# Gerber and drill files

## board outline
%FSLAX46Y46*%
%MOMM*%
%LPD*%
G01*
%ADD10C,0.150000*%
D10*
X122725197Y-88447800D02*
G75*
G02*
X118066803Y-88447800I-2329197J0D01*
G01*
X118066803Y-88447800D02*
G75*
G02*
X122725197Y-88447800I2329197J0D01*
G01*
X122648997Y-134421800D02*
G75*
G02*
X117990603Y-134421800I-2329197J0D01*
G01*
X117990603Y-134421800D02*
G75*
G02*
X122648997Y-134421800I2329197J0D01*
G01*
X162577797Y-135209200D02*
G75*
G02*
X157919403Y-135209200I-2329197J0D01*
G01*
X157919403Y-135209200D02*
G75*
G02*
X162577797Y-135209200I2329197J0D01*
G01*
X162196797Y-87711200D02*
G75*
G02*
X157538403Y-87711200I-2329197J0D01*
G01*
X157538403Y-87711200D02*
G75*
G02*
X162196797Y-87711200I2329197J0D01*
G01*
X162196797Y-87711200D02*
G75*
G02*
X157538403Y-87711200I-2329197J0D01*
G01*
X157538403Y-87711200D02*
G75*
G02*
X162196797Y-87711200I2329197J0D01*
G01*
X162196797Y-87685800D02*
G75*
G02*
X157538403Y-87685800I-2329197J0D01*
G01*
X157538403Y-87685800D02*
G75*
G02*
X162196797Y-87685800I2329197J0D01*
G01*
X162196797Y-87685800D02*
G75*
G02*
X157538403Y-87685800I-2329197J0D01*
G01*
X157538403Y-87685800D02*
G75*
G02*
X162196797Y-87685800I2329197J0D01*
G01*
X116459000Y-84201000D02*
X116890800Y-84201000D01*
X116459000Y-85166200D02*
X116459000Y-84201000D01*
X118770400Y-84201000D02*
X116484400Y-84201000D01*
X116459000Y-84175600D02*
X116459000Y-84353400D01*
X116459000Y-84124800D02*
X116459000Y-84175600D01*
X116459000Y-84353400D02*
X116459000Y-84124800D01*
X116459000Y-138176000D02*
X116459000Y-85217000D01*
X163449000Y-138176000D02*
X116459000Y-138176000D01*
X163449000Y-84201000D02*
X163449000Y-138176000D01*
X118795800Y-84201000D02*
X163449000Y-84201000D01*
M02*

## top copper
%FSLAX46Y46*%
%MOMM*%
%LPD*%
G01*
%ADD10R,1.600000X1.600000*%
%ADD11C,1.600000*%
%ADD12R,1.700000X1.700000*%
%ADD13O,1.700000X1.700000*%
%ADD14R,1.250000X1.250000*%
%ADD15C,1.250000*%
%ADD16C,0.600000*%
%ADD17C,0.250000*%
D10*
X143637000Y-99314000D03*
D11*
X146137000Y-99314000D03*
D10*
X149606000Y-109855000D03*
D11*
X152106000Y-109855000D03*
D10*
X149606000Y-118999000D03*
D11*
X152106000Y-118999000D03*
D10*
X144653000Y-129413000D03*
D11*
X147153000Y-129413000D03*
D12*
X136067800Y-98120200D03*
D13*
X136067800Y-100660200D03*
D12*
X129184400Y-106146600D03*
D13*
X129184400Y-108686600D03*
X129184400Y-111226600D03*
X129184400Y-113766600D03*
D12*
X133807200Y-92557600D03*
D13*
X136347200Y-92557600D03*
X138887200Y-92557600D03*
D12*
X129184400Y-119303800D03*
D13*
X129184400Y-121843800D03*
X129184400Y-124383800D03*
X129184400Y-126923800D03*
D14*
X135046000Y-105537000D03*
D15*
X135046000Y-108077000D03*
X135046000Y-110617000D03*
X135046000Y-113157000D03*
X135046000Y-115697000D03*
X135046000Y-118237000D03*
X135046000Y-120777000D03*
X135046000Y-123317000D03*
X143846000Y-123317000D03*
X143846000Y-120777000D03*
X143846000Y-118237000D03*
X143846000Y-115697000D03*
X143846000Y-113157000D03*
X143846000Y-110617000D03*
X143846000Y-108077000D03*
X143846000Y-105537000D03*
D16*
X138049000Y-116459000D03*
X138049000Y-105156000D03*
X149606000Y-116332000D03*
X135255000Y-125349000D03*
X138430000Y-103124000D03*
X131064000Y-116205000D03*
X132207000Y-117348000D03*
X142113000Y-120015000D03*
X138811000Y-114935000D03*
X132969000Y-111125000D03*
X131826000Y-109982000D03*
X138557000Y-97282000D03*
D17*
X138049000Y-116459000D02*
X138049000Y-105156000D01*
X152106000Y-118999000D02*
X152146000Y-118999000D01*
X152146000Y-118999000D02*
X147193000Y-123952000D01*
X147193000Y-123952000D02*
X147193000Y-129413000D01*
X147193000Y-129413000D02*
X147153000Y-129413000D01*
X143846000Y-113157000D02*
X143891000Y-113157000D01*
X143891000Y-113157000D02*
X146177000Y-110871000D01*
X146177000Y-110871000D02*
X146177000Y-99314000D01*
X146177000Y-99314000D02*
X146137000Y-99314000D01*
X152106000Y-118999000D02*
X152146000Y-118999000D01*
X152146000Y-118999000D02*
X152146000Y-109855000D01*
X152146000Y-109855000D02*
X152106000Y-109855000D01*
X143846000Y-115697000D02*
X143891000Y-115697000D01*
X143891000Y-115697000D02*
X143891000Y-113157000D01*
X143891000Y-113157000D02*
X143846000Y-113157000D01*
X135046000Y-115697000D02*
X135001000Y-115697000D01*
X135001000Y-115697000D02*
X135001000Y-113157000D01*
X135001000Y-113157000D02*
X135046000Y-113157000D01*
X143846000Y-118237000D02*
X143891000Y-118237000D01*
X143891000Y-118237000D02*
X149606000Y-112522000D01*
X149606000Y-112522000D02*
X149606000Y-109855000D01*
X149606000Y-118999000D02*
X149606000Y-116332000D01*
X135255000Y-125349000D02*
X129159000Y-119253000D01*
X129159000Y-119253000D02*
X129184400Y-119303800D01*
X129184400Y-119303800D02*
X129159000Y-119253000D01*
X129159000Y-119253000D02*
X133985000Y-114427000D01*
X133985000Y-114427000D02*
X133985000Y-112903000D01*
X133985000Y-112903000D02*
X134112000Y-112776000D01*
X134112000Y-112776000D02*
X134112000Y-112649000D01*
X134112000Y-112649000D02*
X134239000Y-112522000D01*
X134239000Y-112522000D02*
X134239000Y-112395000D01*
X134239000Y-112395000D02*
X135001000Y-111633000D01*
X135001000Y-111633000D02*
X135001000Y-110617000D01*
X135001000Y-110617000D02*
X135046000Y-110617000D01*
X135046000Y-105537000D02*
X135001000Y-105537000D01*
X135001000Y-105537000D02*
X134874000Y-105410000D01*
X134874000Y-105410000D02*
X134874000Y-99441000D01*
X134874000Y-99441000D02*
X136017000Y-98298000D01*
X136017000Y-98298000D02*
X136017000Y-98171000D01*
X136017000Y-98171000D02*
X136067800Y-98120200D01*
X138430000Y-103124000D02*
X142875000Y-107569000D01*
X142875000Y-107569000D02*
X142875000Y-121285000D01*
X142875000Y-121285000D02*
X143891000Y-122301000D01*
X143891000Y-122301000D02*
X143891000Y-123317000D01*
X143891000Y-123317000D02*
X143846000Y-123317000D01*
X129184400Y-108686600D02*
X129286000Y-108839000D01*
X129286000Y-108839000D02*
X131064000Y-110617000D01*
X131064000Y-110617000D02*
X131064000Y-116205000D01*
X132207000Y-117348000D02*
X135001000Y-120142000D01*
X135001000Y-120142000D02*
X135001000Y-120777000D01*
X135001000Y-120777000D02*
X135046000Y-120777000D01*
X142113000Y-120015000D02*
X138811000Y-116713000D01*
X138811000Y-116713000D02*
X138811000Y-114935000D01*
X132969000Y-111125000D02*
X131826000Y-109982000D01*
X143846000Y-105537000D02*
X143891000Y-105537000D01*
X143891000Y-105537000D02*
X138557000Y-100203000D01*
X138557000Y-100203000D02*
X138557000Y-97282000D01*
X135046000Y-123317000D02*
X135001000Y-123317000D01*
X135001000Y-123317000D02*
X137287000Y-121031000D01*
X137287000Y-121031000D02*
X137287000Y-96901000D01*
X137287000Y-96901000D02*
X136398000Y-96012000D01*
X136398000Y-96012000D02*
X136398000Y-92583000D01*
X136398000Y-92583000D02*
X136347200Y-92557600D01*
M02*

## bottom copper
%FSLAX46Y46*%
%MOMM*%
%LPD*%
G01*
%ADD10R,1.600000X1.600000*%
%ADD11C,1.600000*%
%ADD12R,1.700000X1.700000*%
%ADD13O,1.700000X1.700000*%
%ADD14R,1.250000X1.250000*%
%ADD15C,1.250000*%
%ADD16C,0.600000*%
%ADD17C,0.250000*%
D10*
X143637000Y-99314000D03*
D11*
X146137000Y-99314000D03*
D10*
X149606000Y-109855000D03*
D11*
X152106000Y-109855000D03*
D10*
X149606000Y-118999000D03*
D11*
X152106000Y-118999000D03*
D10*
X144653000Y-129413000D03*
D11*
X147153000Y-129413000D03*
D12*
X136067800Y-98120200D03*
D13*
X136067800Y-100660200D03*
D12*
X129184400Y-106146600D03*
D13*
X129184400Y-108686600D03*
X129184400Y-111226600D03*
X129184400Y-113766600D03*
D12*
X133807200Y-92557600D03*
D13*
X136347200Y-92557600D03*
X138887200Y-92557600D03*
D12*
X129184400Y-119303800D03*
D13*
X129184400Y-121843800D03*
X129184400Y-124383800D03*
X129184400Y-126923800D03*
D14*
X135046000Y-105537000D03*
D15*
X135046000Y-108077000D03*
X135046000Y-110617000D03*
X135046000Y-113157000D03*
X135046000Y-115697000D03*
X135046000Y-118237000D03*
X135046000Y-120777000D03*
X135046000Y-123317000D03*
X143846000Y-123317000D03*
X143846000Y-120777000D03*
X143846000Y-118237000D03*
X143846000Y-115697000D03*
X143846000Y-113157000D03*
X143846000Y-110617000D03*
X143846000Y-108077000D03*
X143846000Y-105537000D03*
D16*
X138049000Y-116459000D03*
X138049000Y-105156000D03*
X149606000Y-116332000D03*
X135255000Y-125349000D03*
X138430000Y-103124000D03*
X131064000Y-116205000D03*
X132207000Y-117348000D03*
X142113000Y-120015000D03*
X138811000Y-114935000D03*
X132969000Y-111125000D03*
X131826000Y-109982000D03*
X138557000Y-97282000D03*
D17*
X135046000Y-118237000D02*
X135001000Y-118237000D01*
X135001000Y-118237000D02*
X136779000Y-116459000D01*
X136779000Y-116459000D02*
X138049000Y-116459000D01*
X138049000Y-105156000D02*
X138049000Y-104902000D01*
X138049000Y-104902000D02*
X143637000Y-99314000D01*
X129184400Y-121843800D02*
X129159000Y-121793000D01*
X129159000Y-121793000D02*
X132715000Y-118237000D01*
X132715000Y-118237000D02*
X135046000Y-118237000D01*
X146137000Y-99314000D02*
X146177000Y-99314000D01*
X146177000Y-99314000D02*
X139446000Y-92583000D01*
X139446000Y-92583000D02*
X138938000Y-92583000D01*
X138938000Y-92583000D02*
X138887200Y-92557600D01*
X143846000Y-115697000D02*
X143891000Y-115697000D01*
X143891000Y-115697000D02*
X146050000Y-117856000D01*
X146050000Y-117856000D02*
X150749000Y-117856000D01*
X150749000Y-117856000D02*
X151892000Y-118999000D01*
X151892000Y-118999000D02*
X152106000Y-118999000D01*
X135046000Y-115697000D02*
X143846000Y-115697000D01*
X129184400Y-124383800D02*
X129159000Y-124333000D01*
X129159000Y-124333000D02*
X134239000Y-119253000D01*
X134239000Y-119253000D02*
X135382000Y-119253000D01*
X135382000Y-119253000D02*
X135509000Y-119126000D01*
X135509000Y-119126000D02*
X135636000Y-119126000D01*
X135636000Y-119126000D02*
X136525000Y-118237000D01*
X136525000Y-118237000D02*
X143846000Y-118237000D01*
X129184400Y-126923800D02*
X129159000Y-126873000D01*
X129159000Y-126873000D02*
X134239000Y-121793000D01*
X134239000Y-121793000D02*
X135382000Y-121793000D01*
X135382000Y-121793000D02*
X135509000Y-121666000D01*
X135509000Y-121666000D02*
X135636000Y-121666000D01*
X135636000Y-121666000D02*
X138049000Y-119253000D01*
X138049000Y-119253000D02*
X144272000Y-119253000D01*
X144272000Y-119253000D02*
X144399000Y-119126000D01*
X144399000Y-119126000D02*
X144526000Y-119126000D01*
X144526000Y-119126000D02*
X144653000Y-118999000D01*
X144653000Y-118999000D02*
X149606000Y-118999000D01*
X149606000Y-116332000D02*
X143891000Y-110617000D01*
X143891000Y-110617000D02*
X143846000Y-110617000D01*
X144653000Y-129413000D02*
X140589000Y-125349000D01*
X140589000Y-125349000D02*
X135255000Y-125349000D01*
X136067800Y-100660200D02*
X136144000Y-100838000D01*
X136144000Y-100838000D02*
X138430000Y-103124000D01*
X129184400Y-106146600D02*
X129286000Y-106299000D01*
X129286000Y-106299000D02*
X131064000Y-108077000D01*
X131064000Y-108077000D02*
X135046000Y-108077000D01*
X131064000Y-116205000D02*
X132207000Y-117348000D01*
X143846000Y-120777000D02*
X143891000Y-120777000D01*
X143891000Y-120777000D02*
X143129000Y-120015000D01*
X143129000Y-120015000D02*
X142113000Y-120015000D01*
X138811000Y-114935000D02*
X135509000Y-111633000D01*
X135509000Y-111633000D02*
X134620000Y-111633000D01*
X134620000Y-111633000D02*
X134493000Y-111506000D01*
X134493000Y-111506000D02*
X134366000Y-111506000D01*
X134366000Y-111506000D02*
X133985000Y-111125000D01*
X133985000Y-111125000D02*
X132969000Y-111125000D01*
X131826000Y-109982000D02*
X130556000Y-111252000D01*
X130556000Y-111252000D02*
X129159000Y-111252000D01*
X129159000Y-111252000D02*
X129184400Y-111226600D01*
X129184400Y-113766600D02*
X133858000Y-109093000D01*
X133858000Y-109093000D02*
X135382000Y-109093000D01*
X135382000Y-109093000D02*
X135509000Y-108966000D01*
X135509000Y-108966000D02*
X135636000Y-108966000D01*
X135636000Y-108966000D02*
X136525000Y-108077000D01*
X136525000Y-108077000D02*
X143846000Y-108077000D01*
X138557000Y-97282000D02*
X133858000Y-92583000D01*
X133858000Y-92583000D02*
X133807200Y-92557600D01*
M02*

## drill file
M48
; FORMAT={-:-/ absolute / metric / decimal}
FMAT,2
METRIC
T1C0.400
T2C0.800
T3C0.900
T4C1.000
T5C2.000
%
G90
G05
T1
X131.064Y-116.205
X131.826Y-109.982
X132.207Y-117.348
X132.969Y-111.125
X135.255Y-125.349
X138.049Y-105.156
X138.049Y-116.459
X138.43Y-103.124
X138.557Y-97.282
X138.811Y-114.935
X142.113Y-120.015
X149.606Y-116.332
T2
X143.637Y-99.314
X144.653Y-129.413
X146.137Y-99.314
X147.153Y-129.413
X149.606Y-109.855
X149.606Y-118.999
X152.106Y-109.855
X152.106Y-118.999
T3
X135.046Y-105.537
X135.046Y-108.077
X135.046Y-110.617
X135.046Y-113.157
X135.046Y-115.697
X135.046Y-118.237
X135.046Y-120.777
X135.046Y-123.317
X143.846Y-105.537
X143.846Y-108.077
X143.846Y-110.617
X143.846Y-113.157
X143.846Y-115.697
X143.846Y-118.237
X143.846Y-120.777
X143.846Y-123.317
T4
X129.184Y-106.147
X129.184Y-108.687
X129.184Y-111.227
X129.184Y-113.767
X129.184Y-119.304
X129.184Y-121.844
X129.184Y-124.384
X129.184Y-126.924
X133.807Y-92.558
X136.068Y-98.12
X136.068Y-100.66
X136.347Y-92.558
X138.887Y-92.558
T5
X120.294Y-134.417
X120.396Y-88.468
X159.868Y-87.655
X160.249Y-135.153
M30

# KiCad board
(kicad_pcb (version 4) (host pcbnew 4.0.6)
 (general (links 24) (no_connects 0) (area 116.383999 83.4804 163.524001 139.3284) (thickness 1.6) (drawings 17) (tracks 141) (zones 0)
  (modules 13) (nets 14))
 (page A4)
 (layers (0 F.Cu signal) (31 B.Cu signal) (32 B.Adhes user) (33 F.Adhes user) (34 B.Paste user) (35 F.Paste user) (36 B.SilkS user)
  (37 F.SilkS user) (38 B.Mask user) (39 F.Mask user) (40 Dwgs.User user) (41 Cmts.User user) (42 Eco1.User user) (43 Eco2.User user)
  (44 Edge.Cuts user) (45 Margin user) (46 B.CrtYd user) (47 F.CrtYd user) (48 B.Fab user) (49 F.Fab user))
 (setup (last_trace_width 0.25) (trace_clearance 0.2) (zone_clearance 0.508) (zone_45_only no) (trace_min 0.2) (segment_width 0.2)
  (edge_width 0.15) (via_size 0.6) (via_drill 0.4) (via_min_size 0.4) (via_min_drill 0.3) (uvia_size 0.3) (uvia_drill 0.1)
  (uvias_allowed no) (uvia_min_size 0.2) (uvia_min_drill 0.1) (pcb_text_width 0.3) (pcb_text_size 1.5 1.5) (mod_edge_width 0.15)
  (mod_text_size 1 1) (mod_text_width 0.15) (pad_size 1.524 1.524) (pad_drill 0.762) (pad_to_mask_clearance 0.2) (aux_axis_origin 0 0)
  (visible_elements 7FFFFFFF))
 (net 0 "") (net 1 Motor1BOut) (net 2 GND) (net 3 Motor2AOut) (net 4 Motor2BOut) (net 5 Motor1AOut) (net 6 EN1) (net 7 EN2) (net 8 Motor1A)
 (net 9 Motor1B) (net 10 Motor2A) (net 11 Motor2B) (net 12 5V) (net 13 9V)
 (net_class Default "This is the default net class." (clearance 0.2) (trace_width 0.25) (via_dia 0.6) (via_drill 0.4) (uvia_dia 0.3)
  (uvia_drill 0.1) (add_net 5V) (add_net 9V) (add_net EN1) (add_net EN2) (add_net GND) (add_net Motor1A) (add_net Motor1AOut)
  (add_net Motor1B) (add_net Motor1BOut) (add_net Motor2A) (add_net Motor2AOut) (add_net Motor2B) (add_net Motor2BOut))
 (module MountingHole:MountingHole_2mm (layer F.Cu) (at 159.8676 87.6554)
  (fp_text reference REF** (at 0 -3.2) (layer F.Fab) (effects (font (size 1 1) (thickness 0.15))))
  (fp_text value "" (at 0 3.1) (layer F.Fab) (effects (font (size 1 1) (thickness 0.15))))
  (pad "" np_thru_hole circle (at 0 0) (size 2 2) (drill 2) (layers *.Cu *.Mask)))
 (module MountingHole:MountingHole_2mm (layer F.Cu) (at 120.396 88.4682)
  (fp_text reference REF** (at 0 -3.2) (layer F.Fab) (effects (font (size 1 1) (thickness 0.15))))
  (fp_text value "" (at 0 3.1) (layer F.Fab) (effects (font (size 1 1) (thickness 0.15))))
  (pad "" np_thru_hole circle (at 0 0) (size 2 2) (drill 2) (layers *.Cu *.Mask)))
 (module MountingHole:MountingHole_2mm (layer F.Cu) (at 120.2944 134.4168)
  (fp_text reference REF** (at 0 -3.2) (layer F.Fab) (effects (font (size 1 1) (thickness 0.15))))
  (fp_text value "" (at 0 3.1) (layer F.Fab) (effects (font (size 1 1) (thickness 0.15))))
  (pad "" np_thru_hole circle (at 0 0) (size 2 2) (drill 2) (layers *.Cu *.Mask)))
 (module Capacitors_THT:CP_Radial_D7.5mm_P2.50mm (layer F.Cu) (at 143.637 99.314)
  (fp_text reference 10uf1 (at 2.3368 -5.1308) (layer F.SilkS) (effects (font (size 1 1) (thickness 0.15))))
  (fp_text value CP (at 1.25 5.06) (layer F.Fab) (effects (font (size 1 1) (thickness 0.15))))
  (pad 1 thru_hole rect (at 0 0) (size 1.6 1.6) (drill 0.8) (layers *.Cu *.Mask) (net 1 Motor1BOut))
  (pad 2 thru_hole circle (at 2.5 0) (size 1.6 1.6) (drill 0.8) (layers *.Cu *.Mask) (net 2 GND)))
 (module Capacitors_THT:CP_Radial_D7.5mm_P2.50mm (layer F.Cu) (at 149.606 109.855)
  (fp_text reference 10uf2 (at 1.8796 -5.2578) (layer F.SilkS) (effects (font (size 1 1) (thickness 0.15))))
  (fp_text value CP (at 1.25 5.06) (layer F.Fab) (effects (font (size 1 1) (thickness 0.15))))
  (pad 1 thru_hole rect (at 0 0) (size 1.6 1.6) (drill 0.8) (layers *.Cu *.Mask) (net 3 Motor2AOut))
  (pad 2 thru_hole circle (at 2.5 0) (size 1.6 1.6) (drill 0.8) (layers *.Cu *.Mask) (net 2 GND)))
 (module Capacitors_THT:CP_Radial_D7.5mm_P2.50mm (layer F.Cu) (at 149.606 118.999)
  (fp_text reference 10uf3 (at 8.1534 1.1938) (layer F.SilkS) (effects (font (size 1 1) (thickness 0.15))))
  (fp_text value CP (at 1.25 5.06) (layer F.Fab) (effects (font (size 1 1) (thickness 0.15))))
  (pad 1 thru_hole rect (at 0 0) (size 1.6 1.6) (drill 0.8) (layers *.Cu *.Mask) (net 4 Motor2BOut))
  (pad 2 thru_hole circle (at 2.5 0) (size 1.6 1.6) (drill 0.8) (layers *.Cu *.Mask) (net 2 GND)))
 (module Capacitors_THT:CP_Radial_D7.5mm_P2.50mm (layer F.Cu) (at 144.653 129.413)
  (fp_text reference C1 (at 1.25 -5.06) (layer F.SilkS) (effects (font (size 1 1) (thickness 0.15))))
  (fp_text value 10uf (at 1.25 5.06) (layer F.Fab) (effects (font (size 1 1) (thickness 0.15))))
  (pad 1 thru_hole rect (at 0 0) (size 1.6 1.6) (drill 0.8) (layers *.Cu *.Mask) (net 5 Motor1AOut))
  (pad 2 thru_hole circle (at 2.5 0) (size 1.6 1.6) (drill 0.8) (layers *.Cu *.Mask) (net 2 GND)))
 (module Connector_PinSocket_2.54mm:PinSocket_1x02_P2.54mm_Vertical (layer F.Cu) (at 136.0678 98.1202)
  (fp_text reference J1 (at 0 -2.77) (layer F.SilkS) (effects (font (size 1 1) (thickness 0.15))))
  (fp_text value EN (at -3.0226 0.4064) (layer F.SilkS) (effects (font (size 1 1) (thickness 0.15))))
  (pad 1 thru_hole rect (at 0 0) (size 1.7 1.7) (drill 1) (layers *.Cu *.Mask) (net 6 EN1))
  (pad 2 thru_hole oval (at 0 2.54) (size 1.7 1.7) (drill 1) (layers *.Cu *.Mask) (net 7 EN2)))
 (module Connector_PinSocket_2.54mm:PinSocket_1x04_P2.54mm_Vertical (layer F.Cu) (at 129.1844 106.1466)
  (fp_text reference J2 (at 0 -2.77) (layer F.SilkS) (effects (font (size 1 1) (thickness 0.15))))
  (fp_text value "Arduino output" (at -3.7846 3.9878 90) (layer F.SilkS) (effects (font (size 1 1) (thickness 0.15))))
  (pad 1 thru_hole rect (at 0 0) (size 1.7 1.7) (drill 1) (layers *.Cu *.Mask) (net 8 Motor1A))
  (pad 2 thru_hole oval (at 0 2.54) (size 1.7 1.7) (drill 1) (layers *.Cu *.Mask) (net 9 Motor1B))
  (pad 3 thru_hole oval (at 0 5.08) (size 1.7 1.7) (drill 1) (layers *.Cu *.Mask) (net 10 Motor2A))
  (pad 4 thru_hole oval (at 0 7.62) (size 1.7 1.7) (drill 1) (layers *.Cu *.Mask) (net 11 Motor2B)))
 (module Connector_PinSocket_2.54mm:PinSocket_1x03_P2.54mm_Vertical (layer F.Cu) (at 133.8072 92.5576 90)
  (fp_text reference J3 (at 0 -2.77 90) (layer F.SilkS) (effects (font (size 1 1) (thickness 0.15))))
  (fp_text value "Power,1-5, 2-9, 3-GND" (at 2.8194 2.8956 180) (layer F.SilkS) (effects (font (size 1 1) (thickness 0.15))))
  (pad 1 thru_hole rect (at 0 0 90) (size 1.7 1.7) (drill 1) (layers *.Cu *.Mask) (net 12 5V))
  (pad 2 thru_hole oval (at 0 2.54 90) (size 1.7 1.7) (drill 1) (layers *.Cu *.Mask) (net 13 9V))
  (pad 3 thru_hole oval (at 0 5.08 90) (size 1.7 1.7) (drill 1) (layers *.Cu *.Mask) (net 2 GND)))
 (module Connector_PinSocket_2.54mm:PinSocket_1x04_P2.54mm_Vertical (layer F.Cu) (at 129.1844 119.3038)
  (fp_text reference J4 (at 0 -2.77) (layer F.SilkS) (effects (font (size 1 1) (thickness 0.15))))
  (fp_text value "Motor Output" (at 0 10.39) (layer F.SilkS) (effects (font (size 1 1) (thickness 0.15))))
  (pad 1 thru_hole rect (at 0 0) (size 1.7 1.7) (drill 1) (layers *.Cu *.Mask) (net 5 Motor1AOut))
  (pad 2 thru_hole oval (at 0 2.54) (size 1.7 1.7) (drill 1) (layers *.Cu *.Mask) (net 1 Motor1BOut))
  (pad 3 thru_hole oval (at 0 5.08) (size 1.7 1.7) (drill 1) (layers *.Cu *.Mask) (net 3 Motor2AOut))
  (pad 4 thru_hole oval (at 0 7.62) (size 1.7 1.7) (drill 1) (layers *.Cu *.Mask) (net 4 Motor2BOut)))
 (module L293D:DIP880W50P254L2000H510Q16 (layer F.Cu) (at 139.446 114.427)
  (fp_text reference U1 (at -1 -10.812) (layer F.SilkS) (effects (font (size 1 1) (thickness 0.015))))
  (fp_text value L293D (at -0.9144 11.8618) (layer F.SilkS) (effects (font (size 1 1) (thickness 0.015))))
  (pad 1 thru_hole rect (at -4.4 -8.89) (size 1.25 1.25) (drill 0.9) (layers *.Cu *.Mask) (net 6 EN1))
  (pad 2 thru_hole circle (at -4.4 -6.35) (size 1.25 1.25) (drill 0.9) (layers *.Cu *.Mask) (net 8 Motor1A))
  (pad 3 thru_hole circle (at -4.4 -3.81) (size 1.25 1.25) (drill 0.9) (layers *.Cu *.Mask) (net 5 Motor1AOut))
  (pad 4 thru_hole circle (at -4.4 -1.27) (size 1.25 1.25) (drill 0.9) (layers *.Cu *.Mask) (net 2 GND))
  (pad 5 thru_hole circle (at -4.4 1.27) (size 1.25 1.25) (drill 0.9) (layers *.Cu *.Mask) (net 2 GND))
  (pad 6 thru_hole circle (at -4.4 3.81) (size 1.25 1.25) (drill 0.9) (layers *.Cu *.Mask) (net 1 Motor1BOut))
  (pad 7 thru_hole circle (at -4.4 6.35) (size 1.25 1.25) (drill 0.9) (layers *.Cu *.Mask) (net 9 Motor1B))
  (pad 8 thru_hole circle (at -4.4 8.89) (size 1.25 1.25) (drill 0.9) (layers *.Cu *.Mask) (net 13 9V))
  (pad 9 thru_hole circle (at 4.4 8.89) (size 1.25 1.25) (drill 0.9) (layers *.Cu *.Mask) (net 7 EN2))
  (pad 10 thru_hole circle (at 4.4 6.35) (size 1.25 1.25) (drill 0.9) (layers *.Cu *.Mask) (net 10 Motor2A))
  (pad 11 thru_hole circle (at 4.4 3.81) (size 1.25 1.25) (drill 0.9) (layers *.Cu *.Mask) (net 3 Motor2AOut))
  (pad 12 thru_hole circle (at 4.4 1.27) (size 1.25 1.25) (drill 0.9) (layers *.Cu *.Mask) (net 2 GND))
  (pad 13 thru_hole circle (at 4.4 -1.27) (size 1.25 1.25) (drill 0.9) (layers *.Cu *.Mask) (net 2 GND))
  (pad 14 thru_hole circle (at 4.4 -3.81) (size 1.25 1.25) (drill 0.9) (layers *.Cu *.Mask) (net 4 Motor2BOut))
  (pad 15 thru_hole circle (at 4.4 -6.35) (size 1.25 1.25) (drill 0.9) (layers *.Cu *.Mask) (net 11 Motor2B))
  (pad 16 thru_hole circle (at 4.4 -8.89) (size 1.25 1.25) (drill 0.9) (layers *.Cu *.Mask) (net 12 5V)))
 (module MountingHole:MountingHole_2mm (layer F.Cu) (at 160.2486 135.1534)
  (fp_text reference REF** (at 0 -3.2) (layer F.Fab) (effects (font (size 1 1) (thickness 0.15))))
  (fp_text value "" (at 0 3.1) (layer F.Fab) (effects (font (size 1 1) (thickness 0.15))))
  (pad "" np_thru_hole circle (at 0 0) (size 2 2) (drill 2) (layers *.Cu *.Mask)))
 (gr_circle (center 120.396 88.4478) (end 119.2022 86.4478) (layer Edge.Cuts) (width 0.15))
 (gr_circle (center 120.3198 134.4218) (end 119.126 132.4218) (layer Edge.Cuts) (width 0.15))
 (gr_circle (center 160.2486 135.2092) (end 159.0548 133.2092) (layer Edge.Cuts) (width 0.15))
 (gr_circle (center 159.8676 87.7112) (end 158.6738 85.7112) (layer Edge.Cuts) (width 0.15))
 (gr_circle (center 159.8676 87.7112) (end 158.6738 85.7112) (layer Edge.Cuts) (width 0.15))
 (gr_circle (center 159.8676 87.6858) (end 158.6738 85.6858) (layer Edge.Cuts) (width 0.15))
 (gr_circle (center 159.8676 87.6858) (end 158.6738 85.6858) (layer Edge.Cuts) (width 0.15))
 (gr_line (start 116.459 84.201) (end 116.8908 84.201) (angle 90) (layer Edge.Cuts) (width 0.15))
 (gr_line (start 116.459 85.1662) (end 116.459 84.201) (angle 90) (layer Edge.Cuts) (width 0.15))
 (gr_line (start 118.7704 84.201) (end 116.4844 84.201) (angle 90) (layer Edge.Cuts) (width 0.15))
 (gr_line (start 116.459 84.1756) (end 116.459 84.3534) (angle 90) (layer Edge.Cuts) (width 0.15))
 (gr_line (start 116.459 84.1248) (end 116.459 84.1756) (angle 90) (layer Edge.Cuts) (width 0.15))
 (gr_line (start 116.459 84.3534) (end 116.459 84.1248) (angle 90) (layer Edge.Cuts) (width 0.15))
 (gr_line (start 116.459 138.176) (end 116.459 85.217) (angle 90) (layer Edge.Cuts) (width 0.15))
 (gr_line (start 163.449 138.176) (end 116.459 138.176) (angle 90) (layer Edge.Cuts) (width 0.15))
 (gr_line (start 163.449 84.201) (end 163.449 138.176) (angle 90) (layer Edge.Cuts) (width 0.15))
 (gr_line (start 118.7958 84.201) (end 163.449 84.201) (angle 90) (layer Edge.Cuts) (width 0.15))
 (segment (start 135.046 118.237) (end 135.001 118.237) (width 0.25) (layer B.Cu) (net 1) (status 80000))
 (segment (start 135.001 118.237) (end 136.779 116.459) (width 0.25) (layer B.Cu) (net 1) (status 80000))
 (segment (start 136.779 116.459) (end 138.049 116.459) (width 0.25) (layer B.Cu) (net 1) (status 80000))
 (via (at 138.049 116.459) (size 0.6) (layers F.Cu B.Cu) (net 1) (status 80000))
 (segment (start 138.049 116.459) (end 138.049 105.156) (width 0.25) (layer F.Cu) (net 1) (status 80000))
 (via (at 138.049 105.156) (size 0.6) (layers F.Cu B.Cu) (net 1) (status 80000))
 (segment (start 138.049 105.156) (end 138.049 104.902) (width 0.25) (layer B.Cu) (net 1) (status 80000))
 (segment (start 138.049 104.902) (end 143.637 99.314) (width 0.25) (layer B.Cu) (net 1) (status 80000))
 (segment (start 129.1844 121.8438) (end 129.159 121.793) (width 0.25) (layer B.Cu) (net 1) (status 80000))
 (segment (start 129.159 121.793) (end 132.715 118.237) (width 0.25) (layer B.Cu) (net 1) (status 80000))
 (segment (start 132.715 118.237) (end 135.046 118.237) (width 0.25) (layer B.Cu) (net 1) (status 80000))
 (segment (start 146.137 99.314) (end 146.177 99.314) (width 0.25) (layer B.Cu) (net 2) (status 80000))
 (segment (start 146.177 99.314) (end 139.446 92.583) (width 0.25) (layer B.Cu) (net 2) (status 80000))
 (segment (start 139.446 92.583) (end 138.938 92.583) (width 0.25) (layer B.Cu) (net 2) (status 80000))
 (segment (start 138.938 92.583) (end 138.8872 92.5576) (width 0.25) (layer B.Cu) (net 2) (status 80000))
 (segment (start 152.106 118.999) (end 152.146 118.999) (width 0.25) (layer F.Cu) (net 2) (status 80000))
 (segment (start 152.146 118.999) (end 147.193 123.952) (width 0.25) (layer F.Cu) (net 2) (status 80000))
 (segment (start 147.193 123.952) (end 147.193 129.413) (width 0.25) (layer F.Cu) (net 2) (status 80000))
 (segment (start 147.193 129.413) (end 147.153 129.413) (width 0.25) (layer F.Cu) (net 2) (status 80000))
 (segment (start 143.846 113.157) (end 143.891 113.157) (width 0.25) (layer F.Cu) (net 2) (status 80000))
 (segment (start 143.891 113.157) (end 146.177 110.871) (width 0.25) (layer F.Cu) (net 2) (status 80000))
 (segment (start 146.177 110.871) (end 146.177 99.314) (width 0.25) (layer F.Cu) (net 2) (status 80000))
 (segment (start 146.177 99.314) (end 146.137 99.314) (width 0.25) (layer F.Cu) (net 2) (status 80000))
 (segment (start 143.846 115.697) (end 143.891 115.697) (width 0.25) (layer B.Cu) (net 2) (status 80000))
 (segment (start 143.891 115.697) (end 146.05 117.856) (width 0.25) (layer B.Cu) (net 2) (status 80000))
 (segment (start 146.05 117.856) (end 150.749 117.856) (width 0.25) (layer B.Cu) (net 2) (status 80000))
 (segment (start 150.749 117.856) (end 151.892 118.999) (width 0.25) (layer B.Cu) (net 2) (status 80000))
 (segment (start 151.892 118.999) (end 152.106 118.999) (width 0.25) (layer B.Cu) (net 2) (status 80000))
 (segment (start 152.106 118.999) (end 152.146 118.999) (width 0.25) (layer F.Cu) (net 2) (status 80000))
 (segment (start 152.146 118.999) (end 152.146 109.855) (width 0.25) (layer F.Cu) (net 2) (status 80000))
 (segment (start 152.146 109.855) (end 152.106 109.855) (width 0.25) (layer F.Cu) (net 2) (status 80000))
 (segment (start 135.046 115.697) (end 143.846 115.697) (width 0.25) (layer B.Cu) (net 2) (status 80000))
 (segment (start 143.846 115.697) (end 143.891 115.697) (width 0.25) (layer F.Cu) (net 2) (status 80000))
 (segment (start 143.891 115.697) (end 143.891 113.157) (width 0.25) (layer F.Cu) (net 2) (status 80000))
 (segment (start 143.891 113.157) (end 143.846 113.157) (width 0.25) (layer F.Cu) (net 2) (status 80000))
 (segment (start 135.046 115.697) (end 135.001 115.697) (width 0.25) (layer F.Cu) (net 2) (status 80000))
 (segment (start 135.001 115.697) (end 135.001 113.157) (width 0.25) (layer F.Cu) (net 2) (status 80000))
 (segment (start 135.001 113.157) (end 135.046 113.157) (width 0.25) (layer F.Cu) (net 2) (status 80000))
 (segment (start 129.1844 124.3838) (end 129.159 124.333) (width 0.25) (layer B.Cu) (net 3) (status 80000))
 (segment (start 129.159 124.333) (end 134.239 119.253) (width 0.25) (layer B.Cu) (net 3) (status 80000))
 (segment (start 134.239 119.253) (end 135.382 119.253) (width 0.25) (layer B.Cu) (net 3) (status 80000))
 (segment (start 135.382 119.253) (end 135.509 119.126) (width 0.25) (layer B.Cu) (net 3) (status 80000))
 (segment (start 135.509 119.126) (end 135.636 119.126) (width 0.25) (layer B.Cu) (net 3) (status 80000))
 (segment (start 135.636 119.126) (end 136.525 118.237) (width 0.25) (layer B.Cu) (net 3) (status 80000))
 (segment (start 136.525 118.237) (end 143.846 118.237) (width 0.25) (layer B.Cu) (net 3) (status 80000))
 (segment (start 143.846 118.237) (end 143.891 118.237) (width 0.25) (layer F.Cu) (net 3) (status 80000))
 (segment (start 143.891 118.237) (end 149.606 112.522) (width 0.25) (layer F.Cu) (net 3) (status 80000))
 (segment (start 149.606 112.522) (end 149.606 109.855) (width 0.25) (layer F.Cu) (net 3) (status 80000))
 (segment (start 129.1844 126.9238) (end 129.159 126.873) (width 0.25) (layer B.Cu) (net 4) (status 80000))
 (segment (start 129.159 126.873) (end 134.239 121.793) (width 0.25) (layer B.Cu) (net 4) (status 80000))
 (segment (start 134.239 121.793) (end 135.382 121.793) (width 0.25) (layer B.Cu) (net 4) (status 80000))
 (segment (start 135.382 121.793) (end 135.509 121.666) (width 0.25) (layer B.Cu) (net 4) (status 80000))
 (segment (start 135.509 121.666) (end 135.636 121.666) (width 0.25) (layer B.Cu) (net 4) (status 80000))
 (segment (start 135.636 121.666) (end 138.049 119.253) (width 0.25) (layer B.Cu) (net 4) (status 80000))
 (segment (start 138.049 119.253) (end 144.272 119.253) (width 0.25) (layer B.Cu) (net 4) (status 80000))
 (segment (start 144.272 119.253) (end 144.399 119.126) (width 0.25) (layer B.Cu) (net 4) (status 80000))
 (segment (start 144.399 119.126) (end 144.526 119.126) (width 0.25) (layer B.Cu) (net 4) (status 80000))
 (segment (start 144.526 119.126) (end 144.653 118.999) (width 0.25) (layer B.Cu) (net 4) (status 80000))
 (segment (start 144.653 118.999) (end 149.606 118.999) (width 0.25) (layer B.Cu) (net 4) (status 80000))
 (segment (start 149.606 118.999) (end 149.606 116.332) (width 0.25) (layer F.Cu) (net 4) (status 80000))
 (via (at 149.606 116.332) (size 0.6) (layers F.Cu B.Cu) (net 4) (status 80000))
 (segment (start 149.606 116.332) (end 143.891 110.617) (width 0.25) (layer B.Cu) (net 4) (status 80000))
 (segment (start 143.891 110.617) (end 143.846 110.617) (width 0.25) (layer B.Cu) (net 4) (status 80000))
 (segment (start 144.653 129.413) (end 140.589 125.349) (width 0.25) (layer B.Cu) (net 5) (status 80000))
 (segment (start 140.589 125.349) (end 135.255 125.349) (width 0.25) (layer B.Cu) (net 5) (status 80000))
 (via (at 135.255 125.349) (size 0.6) (layers F.Cu B.Cu) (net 5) (status 80000))
 (segment (start 135.255 125.349) (end 129.159 119.253) (width 0.25) (layer F.Cu) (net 5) (status 80000))
 (segment (start 129.159 119.253) (end 129.1844 119.3038) (width 0.25) (layer F.Cu) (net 5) (status 80000))
 (segment (start 129.1844 119.3038) (end 129.159 119.253) (width 0.25) (layer F.Cu) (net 5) (status 80000))
 (segment (start 129.159 119.253) (end 133.985 114.427) (width 0.25) (layer F.Cu) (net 5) (status 80000))
 (segment (start 133.985 114.427) (end 133.985 112.903) (width 0.25) (layer F.Cu) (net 5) (status 80000))
 (segment (start 133.985 112.903) (end 134.112 112.776) (width 0.25) (layer F.Cu) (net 5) (status 80000))
 (segment (start 134.112 112.776) (end 134.112 112.649) (width 0.25) (layer F.Cu) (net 5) (status 80000))
 (segment (start 134.112 112.649) (end 134.239 112.522) (width 0.25) (layer F.Cu) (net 5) (status 80000))
 (segment (start 134.239 112.522) (end 134.239 112.395) (width 0.25) (layer F.Cu) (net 5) (status 80000))
 (segment (start 134.239 112.395) (end 135.001 111.633) (width 0.25) (layer F.Cu) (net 5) (status 80000))
 (segment (start 135.001 111.633) (end 135.001 110.617) (width 0.25) (layer F.Cu) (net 5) (status 80000))
 (segment (start 135.001 110.617) (end 135.046 110.617) (width 0.25) (layer F.Cu) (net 5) (status 80000))
 (segment (start 135.046 105.537) (end 135.001 105.537) (width 0.25) (layer F.Cu) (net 6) (status 80000))
 (segment (start 135.001 105.537) (end 134.874 105.41) (width 0.25) (layer F.Cu) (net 6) (status 80000))
 (segment (start 134.874 105.41) (end 134.874 99.441) (width 0.25) (layer F.Cu) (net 6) (status 80000))
 (segment (start 134.874 99.441) (end 136.017 98.298) (width 0.25) (layer F.Cu) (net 6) (status 80000))
 (segment (start 136.017 98.298) (end 136.017 98.171) (width 0.25) (layer F.Cu) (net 6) (status 80000))
 (segment (start 136.017 98.171) (end 136.0678 98.1202) (width 0.25) (layer F.Cu) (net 6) (status 80000))
 (segment (start 136.0678 100.6602) (end 136.144 100.838) (width 0.25) (layer B.Cu) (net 7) (status 80000))
 (segment (start 136.144 100.838) (end 138.43 103.124) (width 0.25) (layer B.Cu) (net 7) (status 80000))
 (via (at 138.43 103.124) (size 0.6) (layers F.Cu B.Cu) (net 7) (status 80000))
 (segment (start 138.43 103.124) (end 142.875 107.569) (width 0.25) (layer F.Cu) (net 7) (status 80000))
 (segment (start 142.875 107.569) (end 142.875 121.285) (width 0.25) (layer F.Cu) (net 7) (status 80000))
 (segment (start 142.875 121.285) (end 143.891 122.301) (width 0.25) (layer F.Cu) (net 7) (status 80000))
 (segment (start 143.891 122.301) (end 143.891 123.317) (width 0.25) (layer F.Cu) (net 7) (status 80000))
 (segment (start 143.891 123.317) (end 143.846 123.317) (width 0.25) (layer F.Cu) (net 7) (status 80000))
 (segment (start 129.1844 106.1466) (end 129.286 106.299) (width 0.25) (layer B.Cu) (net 8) (status 80000))
 (segment (start 129.286 106.299) (end 131.064 108.077) (width 0.25) (layer B.Cu) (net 8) (status 80000))
 (segment (start 131.064 108.077) (end 135.046 108.077) (width 0.25) (layer B.Cu) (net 8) (status 80000))
 (segment (start 129.1844 108.6866) (end 129.286 108.839) (width 0.25) (layer F.Cu) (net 9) (status 80000))
 (segment (start 129.286 108.839) (end 131.064 110.617) (width 0.25) (layer F.Cu) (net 9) (status 80000))
 (segment (start 131.064 110.617) (end 131.064 116.205) (width 0.25) (layer F.Cu) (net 9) (status 80000))
 (via (at 131.064 116.205) (size 0.6) (layers F.Cu B.Cu) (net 9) (status 80000))
 (segment (start 131.064 116.205) (end 132.207 117.348) (width 0.25) (layer B.Cu) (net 9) (status 80000))
 (via (at 132.207 117.348) (size 0.6) (layers F.Cu B.Cu) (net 9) (status 80000))
 (segment (start 132.207 117.348) (end 135.001 120.142) (width 0.25) (layer F.Cu) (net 9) (status 80000))
 (segment (start 135.001 120.142) (end 135.001 120.777) (width 0.25) (layer F.Cu) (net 9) (status 80000))
 (segment (start 135.001 120.777) (end 135.046 120.777) (width 0.25) (layer F.Cu) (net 9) (status 80000))
 (segment (start 143.846 120.777) (end 143.891 120.777) (width 0.25) (layer B.Cu) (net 10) (status 80000))
 (segment (start 143.891 120.777) (end 143.129 120.015) (width 0.25) (layer B.Cu) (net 10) (status 80000))
 (segment (start 143.129 120.015) (end 142.113 120.015) (width 0.25) (layer B.Cu) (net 10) (status 80000))
 (via (at 142.113 120.015) (size 0.6) (layers F.Cu B.Cu) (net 10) (status 80000))
 (segment (start 142.113 120.015) (end 138.811 116.713) (width 0.25) (layer F.Cu) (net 10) (status 80000))
 (segment (start 138.811 116.713) (end 138.811 114.935) (width 0.25) (layer F.Cu) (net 10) (status 80000))
 (via (at 138.811 114.935) (size 0.6) (layers F.Cu B.Cu) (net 10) (status 80000))
 (segment (start 138.811 114.935) (end 135.509 111.633) (width 0.25) (layer B.Cu) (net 10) (status 80000))
 (segment (start 135.509 111.633) (end 134.62 111.633) (width 0.25) (layer B.Cu) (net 10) (status 80000))
 (segment (start 134.62 111.633) (end 134.493 111.506) (width 0.25) (layer B.Cu) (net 10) (status 80000))
 (segment (start 134.493 111.506) (end 134.366 111.506) (width 0.25) (layer B.Cu) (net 10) (status 80000))
 (segment (start 134.366 111.506) (end 133.985 111.125) (width 0.25) (layer B.Cu) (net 10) (status 80000))
 (segment (start 133.985 111.125) (end 132.969 111.125) (width 0.25) (layer B.Cu) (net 10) (status 80000))
 (via (at 132.969 111.125) (size 0.6) (layers F.Cu B.Cu) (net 10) (status 80000))
 (segment (start 132.969 111.125) (end 131.826 109.982) (width 0.25) (layer F.Cu) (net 10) (status 80000))
 (via (at 131.826 109.982) (size 0.6) (layers F.Cu B.Cu) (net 10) (status 80000))
 (segment (start 131.826 109.982) (end 130.556 111.252) (width 0.25) (layer B.Cu) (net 10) (status 80000))
 (segment (start 130.556 111.252) (end 129.159 111.252) (width 0.25) (layer B.Cu) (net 10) (status 80000))
 (segment (start 129.159 111.252) (end 129.1844 111.2266) (width 0.25) (layer B.Cu) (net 10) (status 80000))
 (segment (start 129.1844 113.7666) (end 133.858 109.093) (width 0.25) (layer B.Cu) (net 11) (status 80000))
 (segment (start 133.858 109.093) (end 135.382 109.093) (width 0.25) (layer B.Cu) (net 11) (status 80000))
 (segment (start 135.382 109.093) (end 135.509 108.966) (width 0.25) (layer B.Cu) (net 11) (status 80000))
 (segment (start 135.509 108.966) (end 135.636 108.966) (width 0.25) (layer B.Cu) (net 11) (status 80000))
 (segment (start 135.636 108.966) (end 136.525 108.077) (width 0.25) (layer B.Cu) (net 11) (status 80000))
 (segment (start 136.525 108.077) (end 143.846 108.077) (width 0.25) (layer B.Cu) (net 11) (status 80000))
 (segment (start 143.846 105.537) (end 143.891 105.537) (width 0.25) (layer F.Cu) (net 12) (status 80000))
 (segment (start 143.891 105.537) (end 138.557 100.203) (width 0.25) (layer F.Cu) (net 12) (status 80000))
 (segment (start 138.557 100.203) (end 138.557 97.282) (width 0.25) (layer F.Cu) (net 12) (status 80000))
 (via (at 138.557 97.282) (size 0.6) (layers F.Cu B.Cu) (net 12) (status 80000))
 (segment (start 138.557 97.282) (end 133.858 92.583) (width 0.25) (layer B.Cu) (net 12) (status 80000))
 (segment (start 133.858 92.583) (end 133.8072 92.5576) (width 0.25) (layer B.Cu) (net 12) (status 80000))
 (segment (start 135.046 123.317) (end 135.001 123.317) (width 0.25) (layer F.Cu) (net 13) (status 80000))
 (segment (start 135.001 123.317) (end 137.287 121.031) (width 0.25) (layer F.Cu) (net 13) (status 80000))
 (segment (start 137.287 121.031) (end 137.287 96.901) (width 0.25) (layer F.Cu) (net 13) (status 80000))
 (segment (start 137.287 96.901) (end 136.398 96.012) (width 0.25) (layer F.Cu) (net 13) (status 80000))
 (segment (start 136.398 96.012) (end 136.398 92.583) (width 0.25) (layer F.Cu) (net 13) (status 80000))
 (segment (start 136.398 92.583) (end 136.3472 92.5576) (width 0.25) (layer F.Cu) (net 13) (status 80000)))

